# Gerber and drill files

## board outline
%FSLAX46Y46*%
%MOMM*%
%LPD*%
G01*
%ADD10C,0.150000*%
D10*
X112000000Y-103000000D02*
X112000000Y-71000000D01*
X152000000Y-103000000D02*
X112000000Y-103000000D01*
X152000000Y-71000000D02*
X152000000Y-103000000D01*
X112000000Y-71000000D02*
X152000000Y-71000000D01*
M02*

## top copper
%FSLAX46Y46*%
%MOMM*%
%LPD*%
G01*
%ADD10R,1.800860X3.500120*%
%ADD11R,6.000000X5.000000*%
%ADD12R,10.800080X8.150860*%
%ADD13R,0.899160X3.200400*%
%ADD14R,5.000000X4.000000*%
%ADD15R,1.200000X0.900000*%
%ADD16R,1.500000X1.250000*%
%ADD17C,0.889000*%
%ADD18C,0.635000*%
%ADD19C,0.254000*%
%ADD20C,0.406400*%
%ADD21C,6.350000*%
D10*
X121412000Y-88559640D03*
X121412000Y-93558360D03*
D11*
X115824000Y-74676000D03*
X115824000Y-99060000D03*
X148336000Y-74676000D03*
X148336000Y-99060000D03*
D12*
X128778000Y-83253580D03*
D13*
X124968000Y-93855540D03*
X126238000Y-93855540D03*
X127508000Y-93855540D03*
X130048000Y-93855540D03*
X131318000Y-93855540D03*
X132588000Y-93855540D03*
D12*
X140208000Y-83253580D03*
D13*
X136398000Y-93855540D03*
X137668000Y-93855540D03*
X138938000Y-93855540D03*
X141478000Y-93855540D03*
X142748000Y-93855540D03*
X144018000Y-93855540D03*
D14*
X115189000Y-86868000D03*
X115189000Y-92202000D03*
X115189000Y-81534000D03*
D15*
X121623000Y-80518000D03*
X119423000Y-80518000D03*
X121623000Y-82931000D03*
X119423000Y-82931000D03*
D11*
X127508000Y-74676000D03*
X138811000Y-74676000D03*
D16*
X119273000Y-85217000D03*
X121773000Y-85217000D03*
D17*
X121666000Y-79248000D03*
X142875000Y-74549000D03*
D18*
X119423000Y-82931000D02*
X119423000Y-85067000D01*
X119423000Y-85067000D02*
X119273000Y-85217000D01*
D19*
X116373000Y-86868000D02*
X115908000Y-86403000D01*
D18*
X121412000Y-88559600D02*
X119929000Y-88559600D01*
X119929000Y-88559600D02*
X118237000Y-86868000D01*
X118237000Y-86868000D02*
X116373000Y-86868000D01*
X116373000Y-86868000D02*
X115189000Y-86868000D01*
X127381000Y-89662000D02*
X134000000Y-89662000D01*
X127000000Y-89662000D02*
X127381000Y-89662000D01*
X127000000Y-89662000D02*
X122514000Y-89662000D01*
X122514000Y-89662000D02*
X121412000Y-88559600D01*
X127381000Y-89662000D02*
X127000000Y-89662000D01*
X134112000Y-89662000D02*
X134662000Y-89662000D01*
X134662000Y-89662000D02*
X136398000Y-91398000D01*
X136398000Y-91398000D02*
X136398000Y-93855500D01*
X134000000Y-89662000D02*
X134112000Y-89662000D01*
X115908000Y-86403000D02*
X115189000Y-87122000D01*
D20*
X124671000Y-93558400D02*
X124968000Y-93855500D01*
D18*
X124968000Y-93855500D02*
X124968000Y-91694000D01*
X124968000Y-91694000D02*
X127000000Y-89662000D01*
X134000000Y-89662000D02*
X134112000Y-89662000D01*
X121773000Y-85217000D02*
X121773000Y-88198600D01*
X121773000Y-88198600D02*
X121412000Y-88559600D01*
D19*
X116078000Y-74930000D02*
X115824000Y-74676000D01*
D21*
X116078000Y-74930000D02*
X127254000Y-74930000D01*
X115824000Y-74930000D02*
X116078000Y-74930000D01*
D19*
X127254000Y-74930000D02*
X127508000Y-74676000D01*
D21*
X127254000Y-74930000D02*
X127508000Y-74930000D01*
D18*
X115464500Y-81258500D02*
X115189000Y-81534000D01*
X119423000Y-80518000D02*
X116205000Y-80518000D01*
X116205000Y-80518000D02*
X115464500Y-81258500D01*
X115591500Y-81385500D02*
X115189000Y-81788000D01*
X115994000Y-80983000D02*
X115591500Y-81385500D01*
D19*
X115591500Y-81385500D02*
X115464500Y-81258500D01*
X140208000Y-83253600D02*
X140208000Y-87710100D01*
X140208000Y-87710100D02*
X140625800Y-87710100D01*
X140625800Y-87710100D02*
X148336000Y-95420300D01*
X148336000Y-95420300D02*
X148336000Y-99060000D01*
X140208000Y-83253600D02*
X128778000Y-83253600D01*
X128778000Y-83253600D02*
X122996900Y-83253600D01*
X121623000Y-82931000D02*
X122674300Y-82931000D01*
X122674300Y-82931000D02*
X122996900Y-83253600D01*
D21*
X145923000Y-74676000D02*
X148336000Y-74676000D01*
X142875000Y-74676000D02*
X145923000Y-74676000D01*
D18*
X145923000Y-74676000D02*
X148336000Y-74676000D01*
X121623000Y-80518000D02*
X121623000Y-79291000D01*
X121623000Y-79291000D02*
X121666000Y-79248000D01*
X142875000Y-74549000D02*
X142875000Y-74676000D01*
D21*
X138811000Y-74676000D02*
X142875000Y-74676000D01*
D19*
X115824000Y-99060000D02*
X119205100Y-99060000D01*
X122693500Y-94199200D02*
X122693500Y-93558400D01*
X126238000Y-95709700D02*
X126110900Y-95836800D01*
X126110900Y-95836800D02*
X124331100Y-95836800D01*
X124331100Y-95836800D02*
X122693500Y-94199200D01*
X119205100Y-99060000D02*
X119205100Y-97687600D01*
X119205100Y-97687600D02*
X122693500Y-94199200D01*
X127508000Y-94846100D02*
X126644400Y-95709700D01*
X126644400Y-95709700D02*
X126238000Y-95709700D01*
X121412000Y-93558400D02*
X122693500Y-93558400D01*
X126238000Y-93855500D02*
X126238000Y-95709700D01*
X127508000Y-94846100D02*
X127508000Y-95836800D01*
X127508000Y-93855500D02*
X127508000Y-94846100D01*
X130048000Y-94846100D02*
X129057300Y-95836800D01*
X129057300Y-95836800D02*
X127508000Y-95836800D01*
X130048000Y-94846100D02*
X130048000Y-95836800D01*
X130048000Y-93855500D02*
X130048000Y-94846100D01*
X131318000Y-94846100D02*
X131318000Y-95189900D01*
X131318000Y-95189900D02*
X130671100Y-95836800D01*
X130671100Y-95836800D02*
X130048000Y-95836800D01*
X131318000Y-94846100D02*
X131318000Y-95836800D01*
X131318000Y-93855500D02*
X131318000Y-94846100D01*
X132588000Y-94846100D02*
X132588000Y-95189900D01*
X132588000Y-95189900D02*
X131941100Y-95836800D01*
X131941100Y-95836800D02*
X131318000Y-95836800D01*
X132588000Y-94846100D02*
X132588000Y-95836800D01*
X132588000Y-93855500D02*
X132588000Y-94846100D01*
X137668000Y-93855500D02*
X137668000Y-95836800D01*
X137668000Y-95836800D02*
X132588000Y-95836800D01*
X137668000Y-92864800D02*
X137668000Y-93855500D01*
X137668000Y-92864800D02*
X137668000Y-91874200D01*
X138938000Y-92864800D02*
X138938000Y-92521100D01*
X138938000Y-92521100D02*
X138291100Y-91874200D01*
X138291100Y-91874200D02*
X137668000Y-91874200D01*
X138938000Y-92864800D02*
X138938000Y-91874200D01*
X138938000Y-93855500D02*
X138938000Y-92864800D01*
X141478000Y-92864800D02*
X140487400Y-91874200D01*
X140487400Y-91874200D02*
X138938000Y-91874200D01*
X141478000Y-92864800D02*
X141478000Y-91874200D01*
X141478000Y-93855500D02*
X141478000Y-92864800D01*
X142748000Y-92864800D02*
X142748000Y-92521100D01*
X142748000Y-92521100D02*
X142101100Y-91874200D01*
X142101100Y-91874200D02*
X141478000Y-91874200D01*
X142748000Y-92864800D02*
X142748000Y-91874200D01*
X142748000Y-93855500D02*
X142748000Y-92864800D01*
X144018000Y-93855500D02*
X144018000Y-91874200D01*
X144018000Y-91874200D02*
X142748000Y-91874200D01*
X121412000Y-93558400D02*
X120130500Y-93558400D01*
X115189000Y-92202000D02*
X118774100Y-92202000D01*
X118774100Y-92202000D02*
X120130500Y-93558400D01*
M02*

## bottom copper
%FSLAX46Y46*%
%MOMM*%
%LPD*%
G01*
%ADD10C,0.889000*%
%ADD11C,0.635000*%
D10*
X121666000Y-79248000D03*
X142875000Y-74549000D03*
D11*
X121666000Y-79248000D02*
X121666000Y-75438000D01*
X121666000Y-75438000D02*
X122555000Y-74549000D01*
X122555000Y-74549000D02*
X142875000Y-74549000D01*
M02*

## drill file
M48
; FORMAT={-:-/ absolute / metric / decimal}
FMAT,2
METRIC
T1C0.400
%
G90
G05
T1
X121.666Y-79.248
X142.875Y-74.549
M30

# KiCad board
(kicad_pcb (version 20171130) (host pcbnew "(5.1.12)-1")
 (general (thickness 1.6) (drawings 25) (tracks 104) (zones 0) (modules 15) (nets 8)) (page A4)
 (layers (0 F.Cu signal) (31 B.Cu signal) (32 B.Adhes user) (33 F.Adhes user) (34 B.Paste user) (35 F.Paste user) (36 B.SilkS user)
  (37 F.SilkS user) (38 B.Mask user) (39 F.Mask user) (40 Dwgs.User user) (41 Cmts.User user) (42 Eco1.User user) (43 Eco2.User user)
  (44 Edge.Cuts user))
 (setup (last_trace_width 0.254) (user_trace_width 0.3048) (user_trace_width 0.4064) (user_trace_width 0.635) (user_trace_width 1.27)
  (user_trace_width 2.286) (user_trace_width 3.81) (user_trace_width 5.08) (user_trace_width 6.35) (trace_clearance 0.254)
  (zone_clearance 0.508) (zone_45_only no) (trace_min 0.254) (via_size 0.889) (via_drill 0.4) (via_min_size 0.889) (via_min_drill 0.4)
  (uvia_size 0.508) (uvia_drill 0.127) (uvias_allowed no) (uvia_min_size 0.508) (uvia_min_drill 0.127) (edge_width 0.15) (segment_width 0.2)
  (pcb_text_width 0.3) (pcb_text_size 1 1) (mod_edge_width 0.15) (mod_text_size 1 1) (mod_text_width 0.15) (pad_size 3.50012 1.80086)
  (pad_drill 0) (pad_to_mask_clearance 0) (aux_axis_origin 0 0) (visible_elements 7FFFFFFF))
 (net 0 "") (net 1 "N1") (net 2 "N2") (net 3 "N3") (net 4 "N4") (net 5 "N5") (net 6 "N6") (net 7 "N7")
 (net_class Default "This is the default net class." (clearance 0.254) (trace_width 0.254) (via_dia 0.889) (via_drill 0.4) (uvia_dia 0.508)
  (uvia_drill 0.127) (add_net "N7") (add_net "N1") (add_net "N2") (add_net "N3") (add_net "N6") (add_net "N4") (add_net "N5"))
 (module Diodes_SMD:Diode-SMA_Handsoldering (layer F.Cu) (at 121.412 91.059 270)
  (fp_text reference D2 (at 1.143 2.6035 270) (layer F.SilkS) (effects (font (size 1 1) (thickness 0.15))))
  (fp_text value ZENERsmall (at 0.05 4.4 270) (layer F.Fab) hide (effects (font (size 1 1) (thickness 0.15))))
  (pad 2 smd rect (at -2.49936 0 270) (size 3.50012 1.80086) (layers F.Cu F.Paste F.Mask) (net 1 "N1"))
  (pad 1 smd rect (at 2.49936 0 270) (size 3.50012 1.80086) (layers F.Cu F.Paste F.Mask) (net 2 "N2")))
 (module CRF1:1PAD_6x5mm (layer F.Cu) (at 115.824 74.676)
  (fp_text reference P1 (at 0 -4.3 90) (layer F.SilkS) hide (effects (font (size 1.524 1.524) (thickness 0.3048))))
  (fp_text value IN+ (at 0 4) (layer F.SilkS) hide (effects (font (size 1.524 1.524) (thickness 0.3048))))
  (pad 1 smd rect (at 0 0) (size 6 5) (layers F.Cu F.Paste F.Mask) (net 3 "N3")))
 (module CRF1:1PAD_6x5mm (layer F.Cu) (at 115.824 99.06)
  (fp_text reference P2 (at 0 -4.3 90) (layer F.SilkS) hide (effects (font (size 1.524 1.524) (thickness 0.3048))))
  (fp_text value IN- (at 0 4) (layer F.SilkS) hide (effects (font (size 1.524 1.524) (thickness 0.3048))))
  (pad 1 smd rect (at 0 0) (size 6 5) (layers F.Cu F.Paste F.Mask) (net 2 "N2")))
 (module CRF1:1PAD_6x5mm (layer F.Cu) (at 148.336 74.676)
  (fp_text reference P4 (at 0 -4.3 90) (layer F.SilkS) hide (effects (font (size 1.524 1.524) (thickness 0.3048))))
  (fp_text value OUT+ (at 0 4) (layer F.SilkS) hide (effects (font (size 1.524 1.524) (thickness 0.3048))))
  (pad 1 smd rect (at 0 0) (size 6 5) (layers F.Cu F.Paste F.Mask) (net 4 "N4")))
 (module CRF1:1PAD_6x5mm (layer F.Cu) (at 148.336 99.06)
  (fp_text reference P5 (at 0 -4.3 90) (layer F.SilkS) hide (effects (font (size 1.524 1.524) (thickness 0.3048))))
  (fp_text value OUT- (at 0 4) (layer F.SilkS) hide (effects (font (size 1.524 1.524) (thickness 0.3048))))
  (pad 1 smd rect (at 0 0) (size 6 5) (layers F.Cu F.Paste F.Mask) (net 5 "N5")))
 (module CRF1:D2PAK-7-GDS (layer F.Cu) (at 128.778 89.154)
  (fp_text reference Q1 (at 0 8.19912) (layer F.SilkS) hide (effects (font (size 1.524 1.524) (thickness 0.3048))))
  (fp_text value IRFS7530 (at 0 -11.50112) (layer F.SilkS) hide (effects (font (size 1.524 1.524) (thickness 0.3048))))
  (pad D smd rect (at 0 -5.90042) (size 10.80008 8.15086) (layers F.Cu F.Paste F.Mask) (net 5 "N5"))
  (pad G smd rect (at -3.81 4.70154) (size 0.89916 3.2004) (layers F.Cu F.Paste F.Mask) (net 1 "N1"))
  (pad S smd rect (at -2.54 4.70154) (size 0.89916 3.2004) (layers F.Cu F.Paste F.Mask) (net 2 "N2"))
  (pad S smd rect (at -1.27 4.70154) (size 0.89916 3.2004) (layers F.Cu F.Paste F.Mask) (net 2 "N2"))
  (pad S smd rect (at 1.27 4.70154) (size 0.89916 3.2004) (layers F.Cu F.Paste F.Mask) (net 2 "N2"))
  (pad S smd rect (at 2.54 4.70154) (size 0.89916 3.2004) (layers F.Cu F.Paste F.Mask) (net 2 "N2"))
  (pad S smd rect (at 3.81 4.70154) (size 0.89916 3.2004) (layers F.Cu F.Paste F.Mask) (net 2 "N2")))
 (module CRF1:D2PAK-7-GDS (layer F.Cu) (at 140.208 89.154)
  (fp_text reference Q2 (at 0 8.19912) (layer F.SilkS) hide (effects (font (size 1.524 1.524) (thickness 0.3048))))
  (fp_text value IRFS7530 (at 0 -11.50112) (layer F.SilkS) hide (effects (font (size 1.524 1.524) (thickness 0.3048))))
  (pad D smd rect (at 0 -5.90042) (size 10.80008 8.15086) (layers F.Cu F.Paste F.Mask) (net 5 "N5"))
  (pad G smd rect (at -3.81 4.70154) (size 0.89916 3.2004) (layers F.Cu F.Paste F.Mask) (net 1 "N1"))
  (pad S smd rect (at -2.54 4.70154) (size 0.89916 3.2004) (layers F.Cu F.Paste F.Mask) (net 2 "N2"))
  (pad S smd rect (at -1.27 4.70154) (size 0.89916 3.2004) (layers F.Cu F.Paste F.Mask) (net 2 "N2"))
  (pad S smd rect (at 1.27 4.70154) (size 0.89916 3.2004) (layers F.Cu F.Paste F.Mask) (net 2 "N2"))
  (pad S smd rect (at 2.54 4.70154) (size 0.89916 3.2004) (layers F.Cu F.Paste F.Mask) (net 2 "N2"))
  (pad S smd rect (at 3.81 4.70154) (size 0.89916 3.2004) (layers F.Cu F.Paste F.Mask) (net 2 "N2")))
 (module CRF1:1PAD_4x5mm (layer F.Cu) (at 115.189 86.868 90)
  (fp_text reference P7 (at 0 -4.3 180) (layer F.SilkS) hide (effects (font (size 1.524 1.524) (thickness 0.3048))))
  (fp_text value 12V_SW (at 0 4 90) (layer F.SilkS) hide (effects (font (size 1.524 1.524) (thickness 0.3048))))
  (pad 1 smd rect (at 0 0 90) (size 4 5) (layers F.Cu F.Paste F.Mask) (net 1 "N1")))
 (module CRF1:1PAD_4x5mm (layer F.Cu) (at 115.189 92.202 90)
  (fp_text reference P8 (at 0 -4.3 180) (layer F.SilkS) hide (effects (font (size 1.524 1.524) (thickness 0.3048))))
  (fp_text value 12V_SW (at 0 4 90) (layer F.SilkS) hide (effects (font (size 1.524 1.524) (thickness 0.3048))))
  (pad 1 smd rect (at 0 0 90) (size 4 5) (layers F.Cu F.Paste F.Mask) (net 2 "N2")))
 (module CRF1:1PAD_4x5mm (layer F.Cu) (at 115.189 81.534 90)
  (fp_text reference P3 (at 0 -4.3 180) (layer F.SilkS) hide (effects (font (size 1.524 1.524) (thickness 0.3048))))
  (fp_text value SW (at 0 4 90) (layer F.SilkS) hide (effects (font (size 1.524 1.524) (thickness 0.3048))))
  (pad 1 smd rect (at 0 0 90) (size 4 5) (layers F.Cu F.Paste F.Mask) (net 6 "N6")))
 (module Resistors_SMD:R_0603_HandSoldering (layer F.Cu) (at 120.523 80.518 180)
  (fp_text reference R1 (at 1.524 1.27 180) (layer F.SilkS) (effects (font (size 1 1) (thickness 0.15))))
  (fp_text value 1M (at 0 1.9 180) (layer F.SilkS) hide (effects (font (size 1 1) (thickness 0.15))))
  (pad 1 smd rect (at -1.1 0 180) (size 1.2 0.9) (layers F.Cu F.Paste F.Mask) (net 4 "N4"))
  (pad 2 smd rect (at 1.1 0 180) (size 1.2 0.9) (layers F.Cu F.Paste F.Mask) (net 6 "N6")))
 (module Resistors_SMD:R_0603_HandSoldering (layer F.Cu) (at 120.523 82.931 180)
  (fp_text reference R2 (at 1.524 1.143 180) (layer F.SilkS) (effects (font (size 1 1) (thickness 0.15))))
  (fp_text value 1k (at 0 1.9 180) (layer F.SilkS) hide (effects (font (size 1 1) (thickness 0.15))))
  (pad 1 smd rect (at -1.1 0 180) (size 1.2 0.9) (layers F.Cu F.Paste F.Mask) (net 5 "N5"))
  (pad 2 smd rect (at 1.1 0 180) (size 1.2 0.9) (layers F.Cu F.Paste F.Mask) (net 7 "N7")))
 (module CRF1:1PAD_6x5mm (layer F.Cu) (at 127.508 74.676)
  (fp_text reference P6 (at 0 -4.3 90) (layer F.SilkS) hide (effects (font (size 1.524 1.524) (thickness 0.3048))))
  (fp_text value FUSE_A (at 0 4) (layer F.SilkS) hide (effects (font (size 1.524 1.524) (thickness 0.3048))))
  (pad 1 smd rect (at 0 0) (size 6 5) (layers F.Cu F.Paste F.Mask) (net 3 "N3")))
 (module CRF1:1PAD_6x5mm (layer F.Cu) (at 138.811 74.676)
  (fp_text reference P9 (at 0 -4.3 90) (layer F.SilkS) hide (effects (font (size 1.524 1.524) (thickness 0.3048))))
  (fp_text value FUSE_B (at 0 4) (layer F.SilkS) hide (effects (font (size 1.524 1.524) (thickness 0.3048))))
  (pad 1 smd rect (at 0 0) (size 6 5) (layers F.Cu F.Paste F.Mask) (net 4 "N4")))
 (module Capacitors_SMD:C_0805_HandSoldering (layer F.Cu) (at 120.523 85.217)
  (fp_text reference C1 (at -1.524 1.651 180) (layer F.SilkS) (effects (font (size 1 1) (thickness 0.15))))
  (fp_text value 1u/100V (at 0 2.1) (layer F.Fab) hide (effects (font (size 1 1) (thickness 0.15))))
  (pad 1 smd rect (at -1.25 0) (size 1.5 1.25) (layers F.Cu F.Paste F.Mask) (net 7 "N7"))
  (pad 2 smd rect (at 1.25 0) (size 1.5 1.25) (layers F.Cu F.Paste F.Mask) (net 1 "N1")))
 (gr_line (start 112 103) (end 112 71) (angle 90) (layer Edge.Cuts) (width 0.15))
 (gr_line (start 152 103) (end 112 103) (angle 90) (layer Edge.Cuts) (width 0.15))
 (gr_line (start 152 71) (end 152 103) (angle 90) (layer Edge.Cuts) (width 0.15))
 (gr_line (start 112 71) (end 152 71) (angle 90) (layer Edge.Cuts) (width 0.15))
 (segment (start 119.423 82.931) (end 119.423 85.067) (width 0.635) (layer F.Cu) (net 7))
 (segment (start 119.423 85.067) (end 119.273 85.217) (width 0.635) (layer F.Cu) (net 7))
 (segment (start 116.373 86.868) (end 115.908 86.403) (width 0.254) (layer F.Cu) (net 1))
 (segment (start 121.412 88.5596) (end 119.929 88.5596) (width 0.635) (layer F.Cu) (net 1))
 (segment (start 119.929 88.5596) (end 118.237 86.868) (width 0.635) (layer F.Cu) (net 1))
 (segment (start 118.237 86.868) (end 116.373 86.868) (width 0.635) (layer F.Cu) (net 1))
 (segment (start 116.373 86.868) (end 115.189 86.868) (width 0.635) (layer F.Cu) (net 1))
 (segment (start 127.381 89.662) (end 134 89.662) (width 0.635) (layer F.Cu) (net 1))
 (segment (start 127 89.662) (end 127.381 89.662) (width 0.635) (layer F.Cu) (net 1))
 (segment (start 127 89.662) (end 122.514 89.662) (width 0.635) (layer F.Cu) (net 1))
 (segment (start 122.514 89.662) (end 121.412 88.5596) (width 0.635) (layer F.Cu) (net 1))
 (segment (start 127.381 89.662) (end 127 89.662) (width 0.635) (layer F.Cu) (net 1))
 (segment (start 134.112 89.662) (end 134.662 89.662) (width 0.635) (layer F.Cu) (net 1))
 (segment (start 134.662 89.662) (end 136.398 91.398) (width 0.635) (layer F.Cu) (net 1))
 (segment (start 136.398 91.398) (end 136.398 93.8555) (width 0.635) (layer F.Cu) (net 1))
 (segment (start 134 89.662) (end 134.112 89.662) (width 0.635) (layer F.Cu) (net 1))
 (segment (start 115.908 86.403) (end 115.189 87.122) (width 0.635) (layer F.Cu) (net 1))
 (segment (start 124.671 93.5584) (end 124.968 93.8555) (width 0.4064) (layer F.Cu) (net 1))
 (segment (start 124.968 93.8555) (end 124.968 91.694) (width 0.635) (layer F.Cu) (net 1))
 (segment (start 124.968 91.694) (end 127 89.662) (width 0.635) (layer F.Cu) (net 1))
 (segment (start 134 89.662) (end 134.112 89.662) (width 0.635) (layer F.Cu) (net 1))
 (segment (start 121.773 85.217) (end 121.773 88.1986) (width 0.635) (layer F.Cu) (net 1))
 (segment (start 121.773 88.1986) (end 121.412 88.5596) (width 0.635) (layer F.Cu) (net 1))
 (segment (start 116.078 74.93) (end 115.824 74.676) (width 0.254) (layer F.Cu) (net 3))
 (segment (start 116.078 74.93) (end 127.254 74.93) (width 6.35) (layer F.Cu) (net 3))
 (segment (start 115.824 74.93) (end 116.078 74.93) (width 6.35) (layer F.Cu) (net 3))
 (segment (start 127.254 74.93) (end 127.508 74.676) (width 0.254) (layer F.Cu) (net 3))
 (segment (start 127.254 74.93) (end 127.508 74.93) (width 6.35) (layer F.Cu) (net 3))
 (segment (start 115.4645 81.2585) (end 115.189 81.534) (width 0.635) (layer F.Cu) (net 6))
 (segment (start 119.423 80.518) (end 116.205 80.518) (width 0.635) (layer F.Cu) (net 6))
 (segment (start 116.205 80.518) (end 115.4645 81.2585) (width 0.635) (layer F.Cu) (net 6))
 (segment (start 115.5915 81.3855) (end 115.189 81.788) (width 0.635) (layer F.Cu) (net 6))
 (segment (start 115.994 80.983) (end 115.5915 81.3855) (width 0.635) (layer F.Cu) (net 6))
 (segment (start 115.5915 81.3855) (end 115.4645 81.2585) (width 0.254) (layer F.Cu) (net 6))
 (segment (start 140.208 83.2536) (end 140.208 87.7101) (width 0.254) (layer F.Cu) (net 5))
 (segment (start 140.208 87.7101) (end 140.6258 87.7101) (width 0.254) (layer F.Cu) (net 5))
 (segment (start 140.6258 87.7101) (end 148.336 95.4203) (width 0.254) (layer F.Cu) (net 5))
 (segment (start 148.336 95.4203) (end 148.336 99.06) (width 0.254) (layer F.Cu) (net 5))
 (segment (start 140.208 83.2536) (end 128.778 83.2536) (width 0.254) (layer F.Cu) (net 5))
 (segment (start 128.778 83.2536) (end 122.9969 83.2536) (width 0.254) (layer F.Cu) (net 5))
 (segment (start 121.623 82.931) (end 122.6743 82.931) (width 0.254) (layer F.Cu) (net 5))
 (segment (start 122.6743 82.931) (end 122.9969 83.2536) (width 0.254) (layer F.Cu) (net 5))
 (segment (start 145.923 74.676) (end 148.336 74.676) (width 6.35) (layer F.Cu) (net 4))
 (segment (start 142.875 74.676) (end 145.923 74.676) (width 6.35) (layer F.Cu) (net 4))
 (segment (start 145.923 74.676) (end 148.336 74.676) (width 0.635) (layer F.Cu) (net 4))
 (segment (start 121.623 80.518) (end 121.623 79.291) (width 0.635) (layer F.Cu) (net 4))
 (segment (start 121.623 79.291) (end 121.666 79.248) (width 0.635) (layer F.Cu) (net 4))
 (segment (start 121.666 79.248) (end 121.666 75.438) (width 0.635) (layer B.Cu) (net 4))
 (segment (start 121.666 75.438) (end 122.555 74.549) (width 0.635) (layer B.Cu) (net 4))
 (segment (start 122.555 74.549) (end 142.875 74.549) (width 0.635) (layer B.Cu) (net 4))
 (segment (start 142.875 74.549) (end 142.875 74.676) (width 0.635) (layer F.Cu) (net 4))
 (segment (start 138.811 74.676) (end 142.875 74.676) (width 6.35) (layer F.Cu) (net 4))
 (via (at 121.666 79.248) (size 0.889) (layers F.Cu B.Cu) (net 4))
 (via (at 142.875 74.549) (size 0.889) (layers F.Cu B.Cu) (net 4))
 (segment (start 115.824 99.06) (end 119.2051 99.06) (width 0.254) (layer F.Cu) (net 2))
 (segment (start 122.6935 94.1992) (end 122.6935 93.5584) (width 0.254) (layer F.Cu) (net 2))
 (segment (start 126.238 95.7097) (end 126.1109 95.8368) (width 0.254) (layer F.Cu) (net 2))
 (segment (start 126.1109 95.8368) (end 124.3311 95.8368) (width 0.254) (layer F.Cu) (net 2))
 (segment (start 124.3311 95.8368) (end 122.6935 94.1992) (width 0.254) (layer F.Cu) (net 2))
 (segment (start 119.2051 99.06) (end 119.2051 97.6876) (width 0.254) (layer F.Cu) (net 2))
 (segment (start 119.2051 97.6876) (end 122.6935 94.1992) (width 0.254) (layer F.Cu) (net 2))
 (segment (start 127.508 94.8461) (end 126.6444 95.7097) (width 0.254) (layer F.Cu) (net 2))
 (segment (start 126.6444 95.7097) (end 126.238 95.7097) (width 0.254) (layer F.Cu) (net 2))
 (segment (start 121.412 93.5584) (end 122.6935 93.5584) (width 0.254) (layer F.Cu) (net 2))
 (segment (start 126.238 93.8555) (end 126.238 95.7097) (width 0.254) (layer F.Cu) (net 2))
 (segment (start 127.508 94.8461) (end 127.508 95.8368) (width 0.254) (layer F.Cu) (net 2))
 (segment (start 127.508 93.8555) (end 127.508 94.8461) (width 0.254) (layer F.Cu) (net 2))
 (segment (start 130.048 94.8461) (end 129.0573 95.8368) (width 0.254) (layer F.Cu) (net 2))
 (segment (start 129.0573 95.8368) (end 127.508 95.8368) (width 0.254) (layer F.Cu) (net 2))
 (segment (start 130.048 94.8461) (end 130.048 95.8368) (width 0.254) (layer F.Cu) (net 2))
 (segment (start 130.048 93.8555) (end 130.048 94.8461) (width 0.254) (layer F.Cu) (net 2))
 (segment (start 131.318 94.8461) (end 131.318 95.1899) (width 0.254) (layer F.Cu) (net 2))
 (segment (start 131.318 95.1899) (end 130.6711 95.8368) (width 0.254) (layer F.Cu) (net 2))
 (segment (start 130.6711 95.8368) (end 130.048 95.8368) (width 0.254) (layer F.Cu) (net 2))
 (segment (start 131.318 94.8461) (end 131.318 95.8368) (width 0.254) (layer F.Cu) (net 2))
 (segment (start 131.318 93.8555) (end 131.318 94.8461) (width 0.254) (layer F.Cu) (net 2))
 (segment (start 132.588 94.8461) (end 132.588 95.1899) (width 0.254) (layer F.Cu) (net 2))
 (segment (start 132.588 95.1899) (end 131.9411 95.8368) (width 0.254) (layer F.Cu) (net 2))
 (segment (start 131.9411 95.8368) (end 131.318 95.8368) (width 0.254) (layer F.Cu) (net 2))
 (segment (start 132.588 94.8461) (end 132.588 95.8368) (width 0.254) (layer F.Cu) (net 2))
 (segment (start 132.588 93.8555) (end 132.588 94.8461) (width 0.254) (layer F.Cu) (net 2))
 (segment (start 137.668 93.8555) (end 137.668 95.8368) (width 0.254) (layer F.Cu) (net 2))
 (segment (start 137.668 95.8368) (end 132.588 95.8368) (width 0.254) (layer F.Cu) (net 2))
 (segment (start 137.668 92.8648) (end 137.668 93.8555) (width 0.254) (layer F.Cu) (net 2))
 (segment (start 137.668 92.8648) (end 137.668 91.8742) (width 0.254) (layer F.Cu) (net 2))
 (segment (start 138.938 92.8648) (end 138.938 92.5211) (width 0.254) (layer F.Cu) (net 2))
 (segment (start 138.938 92.5211) (end 138.2911 91.8742) (width 0.254) (layer F.Cu) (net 2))
 (segment (start 138.2911 91.8742) (end 137.668 91.8742) (width 0.254) (layer F.Cu) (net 2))
 (segment (start 138.938 92.8648) (end 138.938 91.8742) (width 0.254) (layer F.Cu) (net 2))
 (segment (start 138.938 93.8555) (end 138.938 92.8648) (width 0.254) (layer F.Cu) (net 2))
 (segment (start 141.478 92.8648) (end 140.4874 91.8742) (width 0.254) (layer F.Cu) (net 2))
 (segment (start 140.4874 91.8742) (end 138.938 91.8742) (width 0.254) (layer F.Cu) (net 2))
 (segment (start 141.478 92.8648) (end 141.478 91.8742) (width 0.254) (layer F.Cu) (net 2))
 (segment (start 141.478 93.8555) (end 141.478 92.8648) (width 0.254) (layer F.Cu) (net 2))
 (segment (start 142.748 92.8648) (end 142.748 92.5211) (width 0.254) (layer F.Cu) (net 2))
 (segment (start 142.748 92.5211) (end 142.1011 91.8742) (width 0.254) (layer F.Cu) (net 2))
 (segment (start 142.1011 91.8742) (end 141.478 91.8742) (width 0.254) (layer F.Cu) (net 2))
 (segment (start 142.748 92.8648) (end 142.748 91.8742) (width 0.254) (layer F.Cu) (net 2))
 (segment (start 142.748 93.8555) (end 142.748 92.8648) (width 0.254) (layer F.Cu) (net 2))
 (segment (start 144.018 93.8555) (end 144.018 91.8742) (width 0.254) (layer F.Cu) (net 2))
 (segment (start 144.018 91.8742) (end 142.748 91.8742) (width 0.254) (layer F.Cu) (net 2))
 (segment (start 121.412 93.5584) (end 120.1305 93.5584) (width 0.254) (layer F.Cu) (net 2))
 (segment (start 115.189 92.202) (end 118.7741 92.202) (width 0.254) (layer F.Cu) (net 2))
 (segment (start 118.7741 92.202) (end 120.1305 93.5584) (width 0.254) (layer F.Cu) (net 2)))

